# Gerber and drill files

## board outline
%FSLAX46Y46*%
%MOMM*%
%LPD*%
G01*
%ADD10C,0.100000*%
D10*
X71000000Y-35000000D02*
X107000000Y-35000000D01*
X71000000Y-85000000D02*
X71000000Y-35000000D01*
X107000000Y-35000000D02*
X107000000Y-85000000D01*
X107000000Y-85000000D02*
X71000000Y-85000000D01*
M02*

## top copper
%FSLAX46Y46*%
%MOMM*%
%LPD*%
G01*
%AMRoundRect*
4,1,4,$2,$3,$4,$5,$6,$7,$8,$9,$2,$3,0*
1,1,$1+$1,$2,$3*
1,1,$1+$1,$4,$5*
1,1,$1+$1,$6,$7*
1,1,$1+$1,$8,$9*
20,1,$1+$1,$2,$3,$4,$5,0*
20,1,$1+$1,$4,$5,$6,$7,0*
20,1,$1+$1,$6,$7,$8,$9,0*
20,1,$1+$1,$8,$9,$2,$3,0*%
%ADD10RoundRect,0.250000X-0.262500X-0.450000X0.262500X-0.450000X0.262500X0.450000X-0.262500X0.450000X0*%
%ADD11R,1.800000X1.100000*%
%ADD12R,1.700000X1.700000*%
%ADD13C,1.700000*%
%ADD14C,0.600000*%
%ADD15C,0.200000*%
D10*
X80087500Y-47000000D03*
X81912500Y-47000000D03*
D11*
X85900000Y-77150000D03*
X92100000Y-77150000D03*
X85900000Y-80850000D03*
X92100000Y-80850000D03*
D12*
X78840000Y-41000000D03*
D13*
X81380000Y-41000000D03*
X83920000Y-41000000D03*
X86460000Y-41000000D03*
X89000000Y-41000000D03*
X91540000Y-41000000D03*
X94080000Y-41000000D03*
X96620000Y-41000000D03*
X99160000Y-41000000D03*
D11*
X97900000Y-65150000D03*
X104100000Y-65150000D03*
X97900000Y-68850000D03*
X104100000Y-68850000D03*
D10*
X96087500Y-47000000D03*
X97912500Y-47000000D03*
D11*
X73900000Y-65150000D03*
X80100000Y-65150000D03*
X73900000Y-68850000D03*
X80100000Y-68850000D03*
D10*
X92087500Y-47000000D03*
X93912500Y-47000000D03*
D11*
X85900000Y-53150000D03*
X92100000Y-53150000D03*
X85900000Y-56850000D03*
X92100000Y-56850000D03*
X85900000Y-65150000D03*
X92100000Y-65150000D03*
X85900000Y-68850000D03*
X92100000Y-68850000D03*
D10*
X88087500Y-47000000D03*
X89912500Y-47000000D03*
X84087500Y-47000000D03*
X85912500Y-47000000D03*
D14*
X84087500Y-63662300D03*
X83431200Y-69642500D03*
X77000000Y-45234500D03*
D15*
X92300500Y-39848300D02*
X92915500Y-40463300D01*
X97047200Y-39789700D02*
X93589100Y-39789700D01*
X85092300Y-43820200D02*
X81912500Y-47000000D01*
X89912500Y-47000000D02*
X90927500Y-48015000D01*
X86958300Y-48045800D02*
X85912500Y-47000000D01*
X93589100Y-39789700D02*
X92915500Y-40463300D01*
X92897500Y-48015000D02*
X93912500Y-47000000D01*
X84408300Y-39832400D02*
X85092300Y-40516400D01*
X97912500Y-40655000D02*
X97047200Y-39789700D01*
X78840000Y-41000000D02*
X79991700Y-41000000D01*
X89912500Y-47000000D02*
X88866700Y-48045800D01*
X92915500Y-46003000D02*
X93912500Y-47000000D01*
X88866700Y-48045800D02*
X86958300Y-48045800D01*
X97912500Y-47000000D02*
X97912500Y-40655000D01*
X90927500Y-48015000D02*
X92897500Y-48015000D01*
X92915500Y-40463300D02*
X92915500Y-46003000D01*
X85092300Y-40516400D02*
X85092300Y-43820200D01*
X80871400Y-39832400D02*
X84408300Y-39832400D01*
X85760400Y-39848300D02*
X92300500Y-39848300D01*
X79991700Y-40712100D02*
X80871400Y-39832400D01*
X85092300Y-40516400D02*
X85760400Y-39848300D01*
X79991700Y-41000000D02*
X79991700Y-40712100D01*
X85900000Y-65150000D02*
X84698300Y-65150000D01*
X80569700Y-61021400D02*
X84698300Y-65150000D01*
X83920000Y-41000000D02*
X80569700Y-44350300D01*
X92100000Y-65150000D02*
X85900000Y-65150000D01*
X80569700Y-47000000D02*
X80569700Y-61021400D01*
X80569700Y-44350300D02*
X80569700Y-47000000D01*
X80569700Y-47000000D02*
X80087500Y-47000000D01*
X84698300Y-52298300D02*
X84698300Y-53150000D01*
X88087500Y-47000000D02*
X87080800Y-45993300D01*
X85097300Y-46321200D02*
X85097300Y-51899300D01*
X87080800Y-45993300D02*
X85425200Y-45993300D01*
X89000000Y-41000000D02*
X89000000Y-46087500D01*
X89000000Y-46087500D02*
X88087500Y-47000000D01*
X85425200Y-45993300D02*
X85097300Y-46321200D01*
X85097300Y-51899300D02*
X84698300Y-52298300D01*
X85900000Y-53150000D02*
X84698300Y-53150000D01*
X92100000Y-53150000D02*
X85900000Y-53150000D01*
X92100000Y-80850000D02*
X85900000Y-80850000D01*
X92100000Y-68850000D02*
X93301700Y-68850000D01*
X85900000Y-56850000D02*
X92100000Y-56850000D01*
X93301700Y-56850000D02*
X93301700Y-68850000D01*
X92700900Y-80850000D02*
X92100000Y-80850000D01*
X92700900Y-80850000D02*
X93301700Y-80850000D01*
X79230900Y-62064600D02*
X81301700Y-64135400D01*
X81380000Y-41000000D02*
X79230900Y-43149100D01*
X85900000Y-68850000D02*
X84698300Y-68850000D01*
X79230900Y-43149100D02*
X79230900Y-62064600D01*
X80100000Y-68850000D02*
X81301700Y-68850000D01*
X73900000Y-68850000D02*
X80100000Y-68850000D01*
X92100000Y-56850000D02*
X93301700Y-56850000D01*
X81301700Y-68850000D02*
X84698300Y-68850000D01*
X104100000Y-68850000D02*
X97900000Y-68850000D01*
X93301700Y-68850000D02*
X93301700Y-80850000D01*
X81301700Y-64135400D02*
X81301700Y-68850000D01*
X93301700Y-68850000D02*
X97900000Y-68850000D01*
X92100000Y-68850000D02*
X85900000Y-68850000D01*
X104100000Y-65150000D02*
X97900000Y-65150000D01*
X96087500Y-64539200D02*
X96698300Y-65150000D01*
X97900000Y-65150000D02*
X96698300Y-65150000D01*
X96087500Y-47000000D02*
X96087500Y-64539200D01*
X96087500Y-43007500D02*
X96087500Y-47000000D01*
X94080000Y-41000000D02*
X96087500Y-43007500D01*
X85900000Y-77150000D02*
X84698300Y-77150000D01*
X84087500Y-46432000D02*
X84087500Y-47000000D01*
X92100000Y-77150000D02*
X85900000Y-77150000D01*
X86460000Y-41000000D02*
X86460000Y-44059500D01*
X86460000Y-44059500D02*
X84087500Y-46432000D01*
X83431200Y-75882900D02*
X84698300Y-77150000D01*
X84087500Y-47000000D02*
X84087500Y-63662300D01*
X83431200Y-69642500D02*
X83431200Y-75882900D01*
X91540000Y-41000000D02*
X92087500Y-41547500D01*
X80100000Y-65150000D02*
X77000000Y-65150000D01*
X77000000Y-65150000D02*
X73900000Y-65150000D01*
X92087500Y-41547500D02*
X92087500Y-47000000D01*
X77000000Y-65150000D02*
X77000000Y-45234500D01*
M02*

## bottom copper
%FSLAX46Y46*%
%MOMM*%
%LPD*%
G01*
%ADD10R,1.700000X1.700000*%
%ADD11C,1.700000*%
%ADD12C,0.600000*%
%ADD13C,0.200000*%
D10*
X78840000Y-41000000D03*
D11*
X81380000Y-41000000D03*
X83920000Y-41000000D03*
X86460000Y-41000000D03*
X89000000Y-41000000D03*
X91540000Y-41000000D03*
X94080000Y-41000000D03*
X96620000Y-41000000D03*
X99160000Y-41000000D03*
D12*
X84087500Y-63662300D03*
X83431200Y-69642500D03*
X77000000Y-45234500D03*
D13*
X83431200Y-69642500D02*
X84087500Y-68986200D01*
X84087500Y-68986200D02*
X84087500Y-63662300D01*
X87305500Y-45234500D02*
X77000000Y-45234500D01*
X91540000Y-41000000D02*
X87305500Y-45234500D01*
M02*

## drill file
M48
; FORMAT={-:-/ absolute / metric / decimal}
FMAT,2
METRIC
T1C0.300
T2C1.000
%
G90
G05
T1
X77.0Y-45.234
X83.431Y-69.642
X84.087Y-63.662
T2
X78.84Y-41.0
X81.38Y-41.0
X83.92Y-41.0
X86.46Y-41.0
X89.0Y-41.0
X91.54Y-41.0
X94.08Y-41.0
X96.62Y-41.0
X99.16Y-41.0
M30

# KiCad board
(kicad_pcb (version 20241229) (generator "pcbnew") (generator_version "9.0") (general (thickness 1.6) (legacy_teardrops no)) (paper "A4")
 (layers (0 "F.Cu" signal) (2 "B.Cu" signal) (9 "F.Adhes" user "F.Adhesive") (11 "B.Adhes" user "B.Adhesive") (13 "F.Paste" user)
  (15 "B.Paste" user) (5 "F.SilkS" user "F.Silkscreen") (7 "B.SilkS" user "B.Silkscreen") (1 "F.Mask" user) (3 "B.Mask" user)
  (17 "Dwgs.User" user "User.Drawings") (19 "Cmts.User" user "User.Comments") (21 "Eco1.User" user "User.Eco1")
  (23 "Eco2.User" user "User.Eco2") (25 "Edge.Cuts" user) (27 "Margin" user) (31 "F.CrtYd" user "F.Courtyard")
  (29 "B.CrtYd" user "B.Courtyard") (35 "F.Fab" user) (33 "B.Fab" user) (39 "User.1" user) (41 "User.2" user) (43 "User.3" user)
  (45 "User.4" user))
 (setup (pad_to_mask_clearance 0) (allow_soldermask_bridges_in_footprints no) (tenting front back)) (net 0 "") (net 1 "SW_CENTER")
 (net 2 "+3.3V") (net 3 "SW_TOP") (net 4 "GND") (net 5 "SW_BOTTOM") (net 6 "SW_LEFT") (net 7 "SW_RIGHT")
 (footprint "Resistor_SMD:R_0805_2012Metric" (layer "F.Cu") (at 81 47)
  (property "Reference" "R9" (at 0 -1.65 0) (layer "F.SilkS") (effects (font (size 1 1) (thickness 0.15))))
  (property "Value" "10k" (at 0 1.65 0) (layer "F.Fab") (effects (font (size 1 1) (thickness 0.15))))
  (pad "1" smd roundrect (at -0.9125 0) (size 1.025 1.4) (layers "F.Cu" "F.Mask" "F.Paste") (roundrect_rratio 0.243902) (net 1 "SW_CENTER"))
  (pad "2" smd roundrect (at 0.9125 0) (size 1.025 1.4) (layers "F.Cu" "F.Mask" "F.Paste") (roundrect_rratio 0.243902) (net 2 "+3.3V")))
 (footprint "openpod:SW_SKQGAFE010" (layer "F.Cu") (at 89 79)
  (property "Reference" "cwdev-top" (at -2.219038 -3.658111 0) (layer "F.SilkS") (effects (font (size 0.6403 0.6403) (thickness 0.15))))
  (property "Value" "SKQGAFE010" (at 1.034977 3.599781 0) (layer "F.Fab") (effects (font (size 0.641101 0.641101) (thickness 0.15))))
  (pad "1" smd rect (at -3.1 -1.85) (size 1.8 1.1) (layers "F.Cu" "F.Mask" "F.Paste") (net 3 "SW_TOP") (solder_mask_margin 0.102))
  (pad "2" smd rect (at 3.1 -1.85) (size 1.8 1.1) (layers "F.Cu" "F.Mask" "F.Paste") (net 3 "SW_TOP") (solder_mask_margin 0.102))
  (pad "3" smd rect (at -3.1 1.85) (size 1.8 1.1) (layers "F.Cu" "F.Mask" "F.Paste") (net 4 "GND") (solder_mask_margin 0.102))
  (pad "4" smd rect (at 3.1 1.85) (size 1.8 1.1) (layers "F.Cu" "F.Mask" "F.Paste") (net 4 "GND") (solder_mask_margin 0.102))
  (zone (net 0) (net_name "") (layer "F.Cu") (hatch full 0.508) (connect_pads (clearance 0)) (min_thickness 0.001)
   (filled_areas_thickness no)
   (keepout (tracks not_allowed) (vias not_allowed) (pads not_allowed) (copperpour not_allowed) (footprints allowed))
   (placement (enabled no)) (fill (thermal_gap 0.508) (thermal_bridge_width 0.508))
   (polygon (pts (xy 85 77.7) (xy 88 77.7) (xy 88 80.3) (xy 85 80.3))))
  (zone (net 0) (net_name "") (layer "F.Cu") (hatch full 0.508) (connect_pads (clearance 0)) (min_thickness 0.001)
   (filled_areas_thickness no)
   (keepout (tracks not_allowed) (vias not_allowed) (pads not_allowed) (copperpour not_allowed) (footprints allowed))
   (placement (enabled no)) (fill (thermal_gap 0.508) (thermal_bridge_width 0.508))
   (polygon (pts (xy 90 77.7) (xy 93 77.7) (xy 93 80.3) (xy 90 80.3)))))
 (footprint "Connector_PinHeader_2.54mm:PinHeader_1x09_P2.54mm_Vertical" (layer "F.Cu") (at 78.84 41 90)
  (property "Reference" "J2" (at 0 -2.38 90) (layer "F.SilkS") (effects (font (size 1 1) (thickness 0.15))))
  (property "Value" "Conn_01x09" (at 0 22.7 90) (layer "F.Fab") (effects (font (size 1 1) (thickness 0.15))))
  (pad "1" thru_hole rect (at 0 0 90) (size 1.7 1.7) (drill 1) (layers "*.Cu" "*.Mask") (remove_unused_layers no) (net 2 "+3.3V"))
  (pad "2" thru_hole circle (at 0 2.54 90) (size 1.7 1.7) (drill 1) (layers "*.Cu" "*.Mask") (remove_unused_layers no) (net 4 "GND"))
  (pad "3" thru_hole circle (at 0 5.08 90) (size 1.7 1.7) (drill 1) (layers "*.Cu" "*.Mask") (remove_unused_layers no) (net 1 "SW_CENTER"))
  (pad "4" thru_hole circle (at 0 7.62 90) (size 1.7 1.7) (drill 1) (layers "*.Cu" "*.Mask") (remove_unused_layers no) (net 3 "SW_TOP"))
  (pad "5" thru_hole circle (at 0 10.16 90) (size 1.7 1.7) (drill 1) (layers "*.Cu" "*.Mask") (remove_unused_layers no) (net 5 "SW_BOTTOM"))
  (pad "6" thru_hole circle (at 0 12.7 90) (size 1.7 1.7) (drill 1) (layers "*.Cu" "*.Mask") (remove_unused_layers no) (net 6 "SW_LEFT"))
  (pad "7" thru_hole circle (at 0 15.24 90) (size 1.7 1.7) (drill 1) (layers "*.Cu" "*.Mask") (remove_unused_layers no) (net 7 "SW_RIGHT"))
  (pad "8" thru_hole circle (at 0 17.78 90) (size 1.7 1.7) (drill 1) (layers "*.Cu" "*.Mask") (remove_unused_layers no))
  (pad "9" thru_hole circle (at 0 20.32 90) (size 1.7 1.7) (drill 1) (layers "*.Cu" "*.Mask") (remove_unused_layers no)))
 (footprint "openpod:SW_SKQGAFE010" (layer "F.Cu") (at 101 67)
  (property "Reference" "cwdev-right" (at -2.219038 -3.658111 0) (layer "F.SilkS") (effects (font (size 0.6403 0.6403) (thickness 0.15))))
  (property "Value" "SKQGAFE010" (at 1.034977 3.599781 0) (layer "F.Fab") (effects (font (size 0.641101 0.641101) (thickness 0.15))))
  (pad "1" smd rect (at -3.1 -1.85) (size 1.8 1.1) (layers "F.Cu" "F.Mask" "F.Paste") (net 7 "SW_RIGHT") (solder_mask_margin 0.102))
  (pad "2" smd rect (at 3.1 -1.85) (size 1.8 1.1) (layers "F.Cu" "F.Mask" "F.Paste") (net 7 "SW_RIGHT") (solder_mask_margin 0.102))
  (pad "3" smd rect (at -3.1 1.85) (size 1.8 1.1) (layers "F.Cu" "F.Mask" "F.Paste") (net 4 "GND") (solder_mask_margin 0.102))
  (pad "4" smd rect (at 3.1 1.85) (size 1.8 1.1) (layers "F.Cu" "F.Mask" "F.Paste") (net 4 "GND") (solder_mask_margin 0.102))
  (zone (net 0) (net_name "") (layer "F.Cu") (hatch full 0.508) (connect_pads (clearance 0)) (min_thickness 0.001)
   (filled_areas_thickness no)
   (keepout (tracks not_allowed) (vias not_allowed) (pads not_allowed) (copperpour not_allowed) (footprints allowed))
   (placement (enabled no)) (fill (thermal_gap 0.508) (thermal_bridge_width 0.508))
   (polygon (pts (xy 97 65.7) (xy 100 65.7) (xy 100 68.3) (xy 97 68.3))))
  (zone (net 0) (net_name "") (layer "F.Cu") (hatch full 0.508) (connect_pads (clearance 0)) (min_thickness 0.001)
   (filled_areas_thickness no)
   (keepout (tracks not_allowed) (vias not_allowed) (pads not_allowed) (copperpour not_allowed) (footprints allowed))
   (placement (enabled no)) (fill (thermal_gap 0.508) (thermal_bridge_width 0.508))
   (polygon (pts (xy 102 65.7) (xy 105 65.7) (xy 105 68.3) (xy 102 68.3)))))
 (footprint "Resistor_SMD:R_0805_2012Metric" (layer "F.Cu") (at 97 47)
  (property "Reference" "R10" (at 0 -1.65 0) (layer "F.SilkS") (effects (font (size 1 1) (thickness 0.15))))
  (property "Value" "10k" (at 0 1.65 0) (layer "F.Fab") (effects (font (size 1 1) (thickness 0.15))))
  (pad "1" smd roundrect (at -0.9125 0) (size 1.025 1.4) (layers "F.Cu" "F.Mask" "F.Paste") (roundrect_rratio 0.243902) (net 7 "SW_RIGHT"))
  (pad "2" smd roundrect (at 0.9125 0) (size 1.025 1.4) (layers "F.Cu" "F.Mask" "F.Paste") (roundrect_rratio 0.243902) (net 2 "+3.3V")))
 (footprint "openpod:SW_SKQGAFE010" (layer "F.Cu") (at 77 67)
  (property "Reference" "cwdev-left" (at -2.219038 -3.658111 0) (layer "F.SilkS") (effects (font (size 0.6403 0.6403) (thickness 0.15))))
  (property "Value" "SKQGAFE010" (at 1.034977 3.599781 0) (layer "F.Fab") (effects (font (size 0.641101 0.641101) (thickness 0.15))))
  (pad "1" smd rect (at -3.1 -1.85) (size 1.8 1.1) (layers "F.Cu" "F.Mask" "F.Paste") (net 6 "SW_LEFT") (solder_mask_margin 0.102))
  (pad "2" smd rect (at 3.1 -1.85) (size 1.8 1.1) (layers "F.Cu" "F.Mask" "F.Paste") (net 6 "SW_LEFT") (solder_mask_margin 0.102))
  (pad "3" smd rect (at -3.1 1.85) (size 1.8 1.1) (layers "F.Cu" "F.Mask" "F.Paste") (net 4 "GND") (solder_mask_margin 0.102))
  (pad "4" smd rect (at 3.1 1.85) (size 1.8 1.1) (layers "F.Cu" "F.Mask" "F.Paste") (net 4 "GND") (solder_mask_margin 0.102))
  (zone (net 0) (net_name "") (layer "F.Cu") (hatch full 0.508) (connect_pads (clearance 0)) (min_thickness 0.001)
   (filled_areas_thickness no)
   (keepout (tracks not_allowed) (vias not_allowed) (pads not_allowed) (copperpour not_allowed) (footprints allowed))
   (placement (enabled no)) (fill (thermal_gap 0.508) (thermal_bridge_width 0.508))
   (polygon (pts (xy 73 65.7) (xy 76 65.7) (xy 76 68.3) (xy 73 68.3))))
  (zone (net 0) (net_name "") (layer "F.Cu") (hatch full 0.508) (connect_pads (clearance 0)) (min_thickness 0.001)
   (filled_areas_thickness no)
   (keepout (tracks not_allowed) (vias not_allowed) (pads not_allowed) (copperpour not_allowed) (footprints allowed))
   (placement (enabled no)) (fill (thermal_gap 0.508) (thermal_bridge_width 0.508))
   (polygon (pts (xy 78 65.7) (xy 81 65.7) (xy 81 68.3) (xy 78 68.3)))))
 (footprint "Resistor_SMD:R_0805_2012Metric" (layer "F.Cu") (at 93 47)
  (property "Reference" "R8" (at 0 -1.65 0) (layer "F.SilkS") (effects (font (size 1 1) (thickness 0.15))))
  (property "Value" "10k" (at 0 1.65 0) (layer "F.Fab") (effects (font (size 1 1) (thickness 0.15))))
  (pad "1" smd roundrect (at -0.9125 0) (size 1.025 1.4) (layers "F.Cu" "F.Mask" "F.Paste") (roundrect_rratio 0.243902) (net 6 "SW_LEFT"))
  (pad "2" smd roundrect (at 0.9125 0) (size 1.025 1.4) (layers "F.Cu" "F.Mask" "F.Paste") (roundrect_rratio 0.243902) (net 2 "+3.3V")))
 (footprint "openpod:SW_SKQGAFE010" (layer "F.Cu") (at 89 55)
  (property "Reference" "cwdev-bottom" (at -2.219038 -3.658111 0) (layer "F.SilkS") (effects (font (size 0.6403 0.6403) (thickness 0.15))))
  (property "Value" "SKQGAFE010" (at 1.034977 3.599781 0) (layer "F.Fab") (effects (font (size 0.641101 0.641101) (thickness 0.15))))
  (pad "1" smd rect (at -3.1 -1.85) (size 1.8 1.1) (layers "F.Cu" "F.Mask" "F.Paste") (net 5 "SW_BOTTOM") (solder_mask_margin 0.102))
  (pad "2" smd rect (at 3.1 -1.85) (size 1.8 1.1) (layers "F.Cu" "F.Mask" "F.Paste") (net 5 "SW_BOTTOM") (solder_mask_margin 0.102))
  (pad "3" smd rect (at -3.1 1.85) (size 1.8 1.1) (layers "F.Cu" "F.Mask" "F.Paste") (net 4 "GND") (solder_mask_margin 0.102))
  (pad "4" smd rect (at 3.1 1.85) (size 1.8 1.1) (layers "F.Cu" "F.Mask" "F.Paste") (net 4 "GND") (solder_mask_margin 0.102))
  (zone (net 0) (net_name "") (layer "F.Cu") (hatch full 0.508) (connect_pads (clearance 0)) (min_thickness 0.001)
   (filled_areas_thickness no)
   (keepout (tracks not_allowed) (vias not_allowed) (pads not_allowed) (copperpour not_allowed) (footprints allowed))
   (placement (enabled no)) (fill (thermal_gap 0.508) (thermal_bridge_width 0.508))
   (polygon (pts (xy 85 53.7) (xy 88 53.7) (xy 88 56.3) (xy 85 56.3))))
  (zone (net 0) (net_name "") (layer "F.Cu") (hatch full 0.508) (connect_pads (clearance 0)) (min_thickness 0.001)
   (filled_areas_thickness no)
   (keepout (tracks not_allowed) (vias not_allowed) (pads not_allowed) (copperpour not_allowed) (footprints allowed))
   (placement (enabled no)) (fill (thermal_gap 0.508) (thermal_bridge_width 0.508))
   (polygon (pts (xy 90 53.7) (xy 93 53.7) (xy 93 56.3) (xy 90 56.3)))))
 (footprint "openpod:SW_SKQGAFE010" (layer "F.Cu") (at 89 67)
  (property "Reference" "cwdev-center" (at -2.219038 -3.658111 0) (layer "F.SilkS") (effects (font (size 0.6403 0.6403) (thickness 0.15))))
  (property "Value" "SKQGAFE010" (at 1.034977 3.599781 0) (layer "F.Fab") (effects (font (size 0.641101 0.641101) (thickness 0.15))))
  (pad "1" smd rect (at -3.1 -1.85) (size 1.8 1.1) (layers "F.Cu" "F.Mask" "F.Paste") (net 1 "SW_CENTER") (solder_mask_margin 0.102))
  (pad "2" smd rect (at 3.1 -1.85) (size 1.8 1.1) (layers "F.Cu" "F.Mask" "F.Paste") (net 1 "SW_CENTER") (solder_mask_margin 0.102))
  (pad "3" smd rect (at -3.1 1.85) (size 1.8 1.1) (layers "F.Cu" "F.Mask" "F.Paste") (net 4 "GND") (solder_mask_margin 0.102))
  (pad "4" smd rect (at 3.1 1.85) (size 1.8 1.1) (layers "F.Cu" "F.Mask" "F.Paste") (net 4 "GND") (solder_mask_margin 0.102))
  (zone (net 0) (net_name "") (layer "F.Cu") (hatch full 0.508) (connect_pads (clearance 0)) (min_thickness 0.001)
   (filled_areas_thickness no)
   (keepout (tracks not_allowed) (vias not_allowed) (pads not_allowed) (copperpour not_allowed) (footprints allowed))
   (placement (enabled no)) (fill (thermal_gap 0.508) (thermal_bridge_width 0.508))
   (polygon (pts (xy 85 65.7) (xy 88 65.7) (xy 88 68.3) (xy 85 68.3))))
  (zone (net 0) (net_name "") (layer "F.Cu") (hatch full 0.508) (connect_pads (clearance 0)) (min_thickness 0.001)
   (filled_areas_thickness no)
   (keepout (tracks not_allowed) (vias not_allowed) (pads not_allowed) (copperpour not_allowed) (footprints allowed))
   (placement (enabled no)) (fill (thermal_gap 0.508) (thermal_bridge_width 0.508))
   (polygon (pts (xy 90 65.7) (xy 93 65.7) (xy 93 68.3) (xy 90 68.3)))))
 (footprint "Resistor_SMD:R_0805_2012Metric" (layer "F.Cu") (at 89 47)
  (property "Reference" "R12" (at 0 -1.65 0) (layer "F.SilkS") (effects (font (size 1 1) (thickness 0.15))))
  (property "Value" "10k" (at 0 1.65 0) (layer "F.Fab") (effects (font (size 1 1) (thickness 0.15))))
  (pad "1" smd roundrect (at -0.9125 0) (size 1.025 1.4) (layers "F.Cu" "F.Mask" "F.Paste") (roundrect_rratio 0.243902) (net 5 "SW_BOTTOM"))
  (pad "2" smd roundrect (at 0.9125 0) (size 1.025 1.4) (layers "F.Cu" "F.Mask" "F.Paste") (roundrect_rratio 0.243902) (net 2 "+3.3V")))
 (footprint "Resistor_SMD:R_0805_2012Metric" (layer "F.Cu") (at 85 47)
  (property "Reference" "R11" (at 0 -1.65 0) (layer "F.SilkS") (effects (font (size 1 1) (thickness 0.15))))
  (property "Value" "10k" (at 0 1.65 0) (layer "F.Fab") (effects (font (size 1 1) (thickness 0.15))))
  (pad "1" smd roundrect (at -0.9125 0) (size 1.025 1.4) (layers "F.Cu" "F.Mask" "F.Paste") (roundrect_rratio 0.243902) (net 3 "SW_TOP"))
  (pad "2" smd roundrect (at 0.9125 0) (size 1.025 1.4) (layers "F.Cu" "F.Mask" "F.Paste") (roundrect_rratio 0.243902) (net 2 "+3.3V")))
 (gr_line (start 71 35) (end 107 35) (stroke (width 0.1) (type default)) (layer "Edge.Cuts"))
 (gr_line (start 71 85) (end 71 35) (stroke (width 0.1) (type default)) (layer "Edge.Cuts"))
 (gr_line (start 107 35) (end 107 85) (stroke (width 0.1) (type default)) (layer "Edge.Cuts"))
 (gr_line (start 107 85) (end 71 85) (stroke (width 0.1) (type default)) (layer "Edge.Cuts"))
 (segment (start 92.3005 39.8483) (end 92.9155 40.4633) (width 0.2) (layer "F.Cu") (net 2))
 (segment (start 97.0472 39.7897) (end 93.5891 39.7897) (width 0.2) (layer "F.Cu") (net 2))
 (segment (start 85.0923 43.8202) (end 81.9125 47) (width 0.2) (layer "F.Cu") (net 2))
 (segment (start 89.9125 47) (end 90.9275 48.015) (width 0.2) (layer "F.Cu") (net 2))
 (segment (start 86.9583 48.0458) (end 85.9125 47) (width 0.2) (layer "F.Cu") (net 2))
 (segment (start 93.5891 39.7897) (end 92.9155 40.4633) (width 0.2) (layer "F.Cu") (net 2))
 (segment (start 92.8975 48.015) (end 93.9125 47) (width 0.2) (layer "F.Cu") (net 2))
 (segment (start 84.4083 39.8324) (end 85.0923 40.5164) (width 0.2) (layer "F.Cu") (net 2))
 (segment (start 97.9125 40.655) (end 97.0472 39.7897) (width 0.2) (layer "F.Cu") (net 2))
 (segment (start 78.84 41) (end 79.9917 41) (width 0.2) (layer "F.Cu") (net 2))
 (segment (start 89.9125 47) (end 88.8667 48.0458) (width 0.2) (layer "F.Cu") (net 2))
 (segment (start 92.9155 46.003) (end 93.9125 47) (width 0.2) (layer "F.Cu") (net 2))
 (segment (start 88.8667 48.0458) (end 86.9583 48.0458) (width 0.2) (layer "F.Cu") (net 2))
 (segment (start 97.9125 47) (end 97.9125 40.655) (width 0.2) (layer "F.Cu") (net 2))
 (segment (start 90.9275 48.015) (end 92.8975 48.015) (width 0.2) (layer "F.Cu") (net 2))
 (segment (start 92.9155 40.4633) (end 92.9155 46.003) (width 0.2) (layer "F.Cu") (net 2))
 (segment (start 85.0923 40.5164) (end 85.0923 43.8202) (width 0.2) (layer "F.Cu") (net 2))
 (segment (start 80.8714 39.8324) (end 84.4083 39.8324) (width 0.2) (layer "F.Cu") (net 2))
 (segment (start 85.7604 39.8483) (end 92.3005 39.8483) (width 0.2) (layer "F.Cu") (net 2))
 (segment (start 79.9917 40.7121) (end 80.8714 39.8324) (width 0.2) (layer "F.Cu") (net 2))
 (segment (start 85.0923 40.5164) (end 85.7604 39.8483) (width 0.2) (layer "F.Cu") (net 2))
 (segment (start 79.9917 41) (end 79.9917 40.7121) (width 0.2) (layer "F.Cu") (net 2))
 (segment (start 85.9 65.15) (end 84.6983 65.15) (width 0.2) (layer "F.Cu") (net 1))
 (segment (start 80.5697 61.0214) (end 84.6983 65.15) (width 0.2) (layer "F.Cu") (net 1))
 (segment (start 83.92 41) (end 80.5697 44.3503) (width 0.2) (layer "F.Cu") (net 1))
 (segment (start 92.1 65.15) (end 85.9 65.15) (width 0.2) (layer "F.Cu") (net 1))
 (segment (start 80.5697 47) (end 80.5697 61.0214) (width 0.2) (layer "F.Cu") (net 1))
 (segment (start 80.5697 44.3503) (end 80.5697 47) (width 0.2) (layer "F.Cu") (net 1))
 (segment (start 80.5697 47) (end 80.0875 47) (width 0.2) (layer "F.Cu") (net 1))
 (segment (start 84.6983 52.2983) (end 84.6983 53.15) (width 0.2) (layer "F.Cu") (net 5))
 (segment (start 88.0875 47) (end 87.0808 45.9933) (width 0.2) (layer "F.Cu") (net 5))
 (segment (start 85.0973 46.3212) (end 85.0973 51.8993) (width 0.2) (layer "F.Cu") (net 5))
 (segment (start 87.0808 45.9933) (end 85.4252 45.9933) (width 0.2) (layer "F.Cu") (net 5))
 (segment (start 89 41) (end 89 46.0875) (width 0.2) (layer "F.Cu") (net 5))
 (segment (start 89 46.0875) (end 88.0875 47) (width 0.2) (layer "F.Cu") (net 5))
 (segment (start 85.4252 45.9933) (end 85.0973 46.3212) (width 0.2) (layer "F.Cu") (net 5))
 (segment (start 85.0973 51.8993) (end 84.6983 52.2983) (width 0.2) (layer "F.Cu") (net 5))
 (segment (start 85.9 53.15) (end 84.6983 53.15) (width 0.2) (layer "F.Cu") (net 5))
 (segment (start 92.1 53.15) (end 85.9 53.15) (width 0.2) (layer "F.Cu") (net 5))
 (segment (start 92.1 80.85) (end 85.9 80.85) (width 0.2) (layer "F.Cu") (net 4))
 (segment (start 92.1 68.85) (end 93.3017 68.85) (width 0.2) (layer "F.Cu") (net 4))
 (segment (start 85.9 56.85) (end 92.1 56.85) (width 0.2) (layer "F.Cu") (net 4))
 (segment (start 93.3017 56.85) (end 93.3017 68.85) (width 0.2) (layer "F.Cu") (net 4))
 (segment (start 92.7009 80.85) (end 92.1 80.85) (width 0.2) (layer "F.Cu") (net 4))
 (segment (start 92.7009 80.85) (end 93.3017 80.85) (width 0.2) (layer "F.Cu") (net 4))
 (segment (start 79.2309 62.0646) (end 81.3017 64.1354) (width 0.2) (layer "F.Cu") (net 4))
 (segment (start 81.38 41) (end 79.2309 43.1491) (width 0.2) (layer "F.Cu") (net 4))
 (segment (start 85.9 68.85) (end 84.6983 68.85) (width 0.2) (layer "F.Cu") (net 4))
 (segment (start 79.2309 43.1491) (end 79.2309 62.0646) (width 0.2) (layer "F.Cu") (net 4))
 (segment (start 80.1 68.85) (end 81.3017 68.85) (width 0.2) (layer "F.Cu") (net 4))
 (segment (start 73.9 68.85) (end 80.1 68.85) (width 0.2) (layer "F.Cu") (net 4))
 (segment (start 92.1 56.85) (end 93.3017 56.85) (width 0.2) (layer "F.Cu") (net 4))
 (segment (start 81.3017 68.85) (end 84.6983 68.85) (width 0.2) (layer "F.Cu") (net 4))
 (segment (start 104.1 68.85) (end 97.9 68.85) (width 0.2) (layer "F.Cu") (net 4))
 (segment (start 93.3017 68.85) (end 93.3017 80.85) (width 0.2) (layer "F.Cu") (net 4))
 (segment (start 81.3017 64.1354) (end 81.3017 68.85) (width 0.2) (layer "F.Cu") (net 4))
 (segment (start 93.3017 68.85) (end 97.9 68.85) (width 0.2) (layer "F.Cu") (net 4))
 (segment (start 92.1 68.85) (end 85.9 68.85) (width 0.2) (layer "F.Cu") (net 4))
 (segment (start 104.1 65.15) (end 97.9 65.15) (width 0.2) (layer "F.Cu") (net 7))
 (segment (start 96.0875 64.5392) (end 96.6983 65.15) (width 0.2) (layer "F.Cu") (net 7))
 (segment (start 97.9 65.15) (end 96.6983 65.15) (width 0.2) (layer "F.Cu") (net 7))
 (segment (start 96.0875 47) (end 96.0875 64.5392) (width 0.2) (layer "F.Cu") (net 7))
 (segment (start 96.0875 43.0075) (end 96.0875 47) (width 0.2) (layer "F.Cu") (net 7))
 (segment (start 94.08 41) (end 96.0875 43.0075) (width 0.2) (layer "F.Cu") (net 7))
 (segment (start 85.9 77.15) (end 84.6983 77.15) (width 0.2) (layer "F.Cu") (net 3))
 (segment (start 84.0875 46.432) (end 84.0875 47) (width 0.2) (layer "F.Cu") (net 3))
 (segment (start 92.1 77.15) (end 85.9 77.15) (width 0.2) (layer "F.Cu") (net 3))
 (segment (start 86.46 41) (end 86.46 44.0595) (width 0.2) (layer "F.Cu") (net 3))
 (segment (start 86.46 44.0595) (end 84.0875 46.432) (width 0.2) (layer "F.Cu") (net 3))
 (segment (start 83.4312 75.8829) (end 84.6983 77.15) (width 0.2) (layer "F.Cu") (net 3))
 (segment (start 84.0875 47) (end 84.0875 63.6623) (width 0.2) (layer "F.Cu") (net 3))
 (segment (start 83.4312 69.6425) (end 83.4312 75.8829) (width 0.2) (layer "F.Cu") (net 3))
 (via (at 84.0875 63.6623) (size 0.6) (drill 0.3) (layers "F.Cu" "B.Cu") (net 3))
 (via (at 83.4312 69.6425) (size 0.6) (drill 0.3) (layers "F.Cu" "B.Cu") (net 3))
 (segment (start 83.4312 69.6425) (end 84.0875 68.9862) (width 0.2) (layer "B.Cu") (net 3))
 (segment (start 84.0875 68.9862) (end 84.0875 63.6623) (width 0.2) (layer "B.Cu") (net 3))
 (segment (start 91.54 41) (end 92.0875 41.5475) (width 0.2) (layer "F.Cu") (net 6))
 (segment (start 80.1 65.15) (end 77 65.15) (width 0.2) (layer "F.Cu") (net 6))
 (segment (start 77 65.15) (end 73.9 65.15) (width 0.2) (layer "F.Cu") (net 6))
 (segment (start 92.0875 41.5475) (end 92.0875 47) (width 0.2) (layer "F.Cu") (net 6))
 (segment (start 77 65.15) (end 77 45.2345) (width 0.2) (layer "F.Cu") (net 6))
 (via (at 77 45.2345) (size 0.6) (drill 0.3) (layers "F.Cu" "B.Cu") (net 6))
 (segment (start 87.3055 45.2345) (end 77 45.2345) (width 0.2) (layer "B.Cu") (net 6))
 (segment (start 91.54 41) (end 87.3055 45.2345) (width 0.2) (layer "B.Cu") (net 6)))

